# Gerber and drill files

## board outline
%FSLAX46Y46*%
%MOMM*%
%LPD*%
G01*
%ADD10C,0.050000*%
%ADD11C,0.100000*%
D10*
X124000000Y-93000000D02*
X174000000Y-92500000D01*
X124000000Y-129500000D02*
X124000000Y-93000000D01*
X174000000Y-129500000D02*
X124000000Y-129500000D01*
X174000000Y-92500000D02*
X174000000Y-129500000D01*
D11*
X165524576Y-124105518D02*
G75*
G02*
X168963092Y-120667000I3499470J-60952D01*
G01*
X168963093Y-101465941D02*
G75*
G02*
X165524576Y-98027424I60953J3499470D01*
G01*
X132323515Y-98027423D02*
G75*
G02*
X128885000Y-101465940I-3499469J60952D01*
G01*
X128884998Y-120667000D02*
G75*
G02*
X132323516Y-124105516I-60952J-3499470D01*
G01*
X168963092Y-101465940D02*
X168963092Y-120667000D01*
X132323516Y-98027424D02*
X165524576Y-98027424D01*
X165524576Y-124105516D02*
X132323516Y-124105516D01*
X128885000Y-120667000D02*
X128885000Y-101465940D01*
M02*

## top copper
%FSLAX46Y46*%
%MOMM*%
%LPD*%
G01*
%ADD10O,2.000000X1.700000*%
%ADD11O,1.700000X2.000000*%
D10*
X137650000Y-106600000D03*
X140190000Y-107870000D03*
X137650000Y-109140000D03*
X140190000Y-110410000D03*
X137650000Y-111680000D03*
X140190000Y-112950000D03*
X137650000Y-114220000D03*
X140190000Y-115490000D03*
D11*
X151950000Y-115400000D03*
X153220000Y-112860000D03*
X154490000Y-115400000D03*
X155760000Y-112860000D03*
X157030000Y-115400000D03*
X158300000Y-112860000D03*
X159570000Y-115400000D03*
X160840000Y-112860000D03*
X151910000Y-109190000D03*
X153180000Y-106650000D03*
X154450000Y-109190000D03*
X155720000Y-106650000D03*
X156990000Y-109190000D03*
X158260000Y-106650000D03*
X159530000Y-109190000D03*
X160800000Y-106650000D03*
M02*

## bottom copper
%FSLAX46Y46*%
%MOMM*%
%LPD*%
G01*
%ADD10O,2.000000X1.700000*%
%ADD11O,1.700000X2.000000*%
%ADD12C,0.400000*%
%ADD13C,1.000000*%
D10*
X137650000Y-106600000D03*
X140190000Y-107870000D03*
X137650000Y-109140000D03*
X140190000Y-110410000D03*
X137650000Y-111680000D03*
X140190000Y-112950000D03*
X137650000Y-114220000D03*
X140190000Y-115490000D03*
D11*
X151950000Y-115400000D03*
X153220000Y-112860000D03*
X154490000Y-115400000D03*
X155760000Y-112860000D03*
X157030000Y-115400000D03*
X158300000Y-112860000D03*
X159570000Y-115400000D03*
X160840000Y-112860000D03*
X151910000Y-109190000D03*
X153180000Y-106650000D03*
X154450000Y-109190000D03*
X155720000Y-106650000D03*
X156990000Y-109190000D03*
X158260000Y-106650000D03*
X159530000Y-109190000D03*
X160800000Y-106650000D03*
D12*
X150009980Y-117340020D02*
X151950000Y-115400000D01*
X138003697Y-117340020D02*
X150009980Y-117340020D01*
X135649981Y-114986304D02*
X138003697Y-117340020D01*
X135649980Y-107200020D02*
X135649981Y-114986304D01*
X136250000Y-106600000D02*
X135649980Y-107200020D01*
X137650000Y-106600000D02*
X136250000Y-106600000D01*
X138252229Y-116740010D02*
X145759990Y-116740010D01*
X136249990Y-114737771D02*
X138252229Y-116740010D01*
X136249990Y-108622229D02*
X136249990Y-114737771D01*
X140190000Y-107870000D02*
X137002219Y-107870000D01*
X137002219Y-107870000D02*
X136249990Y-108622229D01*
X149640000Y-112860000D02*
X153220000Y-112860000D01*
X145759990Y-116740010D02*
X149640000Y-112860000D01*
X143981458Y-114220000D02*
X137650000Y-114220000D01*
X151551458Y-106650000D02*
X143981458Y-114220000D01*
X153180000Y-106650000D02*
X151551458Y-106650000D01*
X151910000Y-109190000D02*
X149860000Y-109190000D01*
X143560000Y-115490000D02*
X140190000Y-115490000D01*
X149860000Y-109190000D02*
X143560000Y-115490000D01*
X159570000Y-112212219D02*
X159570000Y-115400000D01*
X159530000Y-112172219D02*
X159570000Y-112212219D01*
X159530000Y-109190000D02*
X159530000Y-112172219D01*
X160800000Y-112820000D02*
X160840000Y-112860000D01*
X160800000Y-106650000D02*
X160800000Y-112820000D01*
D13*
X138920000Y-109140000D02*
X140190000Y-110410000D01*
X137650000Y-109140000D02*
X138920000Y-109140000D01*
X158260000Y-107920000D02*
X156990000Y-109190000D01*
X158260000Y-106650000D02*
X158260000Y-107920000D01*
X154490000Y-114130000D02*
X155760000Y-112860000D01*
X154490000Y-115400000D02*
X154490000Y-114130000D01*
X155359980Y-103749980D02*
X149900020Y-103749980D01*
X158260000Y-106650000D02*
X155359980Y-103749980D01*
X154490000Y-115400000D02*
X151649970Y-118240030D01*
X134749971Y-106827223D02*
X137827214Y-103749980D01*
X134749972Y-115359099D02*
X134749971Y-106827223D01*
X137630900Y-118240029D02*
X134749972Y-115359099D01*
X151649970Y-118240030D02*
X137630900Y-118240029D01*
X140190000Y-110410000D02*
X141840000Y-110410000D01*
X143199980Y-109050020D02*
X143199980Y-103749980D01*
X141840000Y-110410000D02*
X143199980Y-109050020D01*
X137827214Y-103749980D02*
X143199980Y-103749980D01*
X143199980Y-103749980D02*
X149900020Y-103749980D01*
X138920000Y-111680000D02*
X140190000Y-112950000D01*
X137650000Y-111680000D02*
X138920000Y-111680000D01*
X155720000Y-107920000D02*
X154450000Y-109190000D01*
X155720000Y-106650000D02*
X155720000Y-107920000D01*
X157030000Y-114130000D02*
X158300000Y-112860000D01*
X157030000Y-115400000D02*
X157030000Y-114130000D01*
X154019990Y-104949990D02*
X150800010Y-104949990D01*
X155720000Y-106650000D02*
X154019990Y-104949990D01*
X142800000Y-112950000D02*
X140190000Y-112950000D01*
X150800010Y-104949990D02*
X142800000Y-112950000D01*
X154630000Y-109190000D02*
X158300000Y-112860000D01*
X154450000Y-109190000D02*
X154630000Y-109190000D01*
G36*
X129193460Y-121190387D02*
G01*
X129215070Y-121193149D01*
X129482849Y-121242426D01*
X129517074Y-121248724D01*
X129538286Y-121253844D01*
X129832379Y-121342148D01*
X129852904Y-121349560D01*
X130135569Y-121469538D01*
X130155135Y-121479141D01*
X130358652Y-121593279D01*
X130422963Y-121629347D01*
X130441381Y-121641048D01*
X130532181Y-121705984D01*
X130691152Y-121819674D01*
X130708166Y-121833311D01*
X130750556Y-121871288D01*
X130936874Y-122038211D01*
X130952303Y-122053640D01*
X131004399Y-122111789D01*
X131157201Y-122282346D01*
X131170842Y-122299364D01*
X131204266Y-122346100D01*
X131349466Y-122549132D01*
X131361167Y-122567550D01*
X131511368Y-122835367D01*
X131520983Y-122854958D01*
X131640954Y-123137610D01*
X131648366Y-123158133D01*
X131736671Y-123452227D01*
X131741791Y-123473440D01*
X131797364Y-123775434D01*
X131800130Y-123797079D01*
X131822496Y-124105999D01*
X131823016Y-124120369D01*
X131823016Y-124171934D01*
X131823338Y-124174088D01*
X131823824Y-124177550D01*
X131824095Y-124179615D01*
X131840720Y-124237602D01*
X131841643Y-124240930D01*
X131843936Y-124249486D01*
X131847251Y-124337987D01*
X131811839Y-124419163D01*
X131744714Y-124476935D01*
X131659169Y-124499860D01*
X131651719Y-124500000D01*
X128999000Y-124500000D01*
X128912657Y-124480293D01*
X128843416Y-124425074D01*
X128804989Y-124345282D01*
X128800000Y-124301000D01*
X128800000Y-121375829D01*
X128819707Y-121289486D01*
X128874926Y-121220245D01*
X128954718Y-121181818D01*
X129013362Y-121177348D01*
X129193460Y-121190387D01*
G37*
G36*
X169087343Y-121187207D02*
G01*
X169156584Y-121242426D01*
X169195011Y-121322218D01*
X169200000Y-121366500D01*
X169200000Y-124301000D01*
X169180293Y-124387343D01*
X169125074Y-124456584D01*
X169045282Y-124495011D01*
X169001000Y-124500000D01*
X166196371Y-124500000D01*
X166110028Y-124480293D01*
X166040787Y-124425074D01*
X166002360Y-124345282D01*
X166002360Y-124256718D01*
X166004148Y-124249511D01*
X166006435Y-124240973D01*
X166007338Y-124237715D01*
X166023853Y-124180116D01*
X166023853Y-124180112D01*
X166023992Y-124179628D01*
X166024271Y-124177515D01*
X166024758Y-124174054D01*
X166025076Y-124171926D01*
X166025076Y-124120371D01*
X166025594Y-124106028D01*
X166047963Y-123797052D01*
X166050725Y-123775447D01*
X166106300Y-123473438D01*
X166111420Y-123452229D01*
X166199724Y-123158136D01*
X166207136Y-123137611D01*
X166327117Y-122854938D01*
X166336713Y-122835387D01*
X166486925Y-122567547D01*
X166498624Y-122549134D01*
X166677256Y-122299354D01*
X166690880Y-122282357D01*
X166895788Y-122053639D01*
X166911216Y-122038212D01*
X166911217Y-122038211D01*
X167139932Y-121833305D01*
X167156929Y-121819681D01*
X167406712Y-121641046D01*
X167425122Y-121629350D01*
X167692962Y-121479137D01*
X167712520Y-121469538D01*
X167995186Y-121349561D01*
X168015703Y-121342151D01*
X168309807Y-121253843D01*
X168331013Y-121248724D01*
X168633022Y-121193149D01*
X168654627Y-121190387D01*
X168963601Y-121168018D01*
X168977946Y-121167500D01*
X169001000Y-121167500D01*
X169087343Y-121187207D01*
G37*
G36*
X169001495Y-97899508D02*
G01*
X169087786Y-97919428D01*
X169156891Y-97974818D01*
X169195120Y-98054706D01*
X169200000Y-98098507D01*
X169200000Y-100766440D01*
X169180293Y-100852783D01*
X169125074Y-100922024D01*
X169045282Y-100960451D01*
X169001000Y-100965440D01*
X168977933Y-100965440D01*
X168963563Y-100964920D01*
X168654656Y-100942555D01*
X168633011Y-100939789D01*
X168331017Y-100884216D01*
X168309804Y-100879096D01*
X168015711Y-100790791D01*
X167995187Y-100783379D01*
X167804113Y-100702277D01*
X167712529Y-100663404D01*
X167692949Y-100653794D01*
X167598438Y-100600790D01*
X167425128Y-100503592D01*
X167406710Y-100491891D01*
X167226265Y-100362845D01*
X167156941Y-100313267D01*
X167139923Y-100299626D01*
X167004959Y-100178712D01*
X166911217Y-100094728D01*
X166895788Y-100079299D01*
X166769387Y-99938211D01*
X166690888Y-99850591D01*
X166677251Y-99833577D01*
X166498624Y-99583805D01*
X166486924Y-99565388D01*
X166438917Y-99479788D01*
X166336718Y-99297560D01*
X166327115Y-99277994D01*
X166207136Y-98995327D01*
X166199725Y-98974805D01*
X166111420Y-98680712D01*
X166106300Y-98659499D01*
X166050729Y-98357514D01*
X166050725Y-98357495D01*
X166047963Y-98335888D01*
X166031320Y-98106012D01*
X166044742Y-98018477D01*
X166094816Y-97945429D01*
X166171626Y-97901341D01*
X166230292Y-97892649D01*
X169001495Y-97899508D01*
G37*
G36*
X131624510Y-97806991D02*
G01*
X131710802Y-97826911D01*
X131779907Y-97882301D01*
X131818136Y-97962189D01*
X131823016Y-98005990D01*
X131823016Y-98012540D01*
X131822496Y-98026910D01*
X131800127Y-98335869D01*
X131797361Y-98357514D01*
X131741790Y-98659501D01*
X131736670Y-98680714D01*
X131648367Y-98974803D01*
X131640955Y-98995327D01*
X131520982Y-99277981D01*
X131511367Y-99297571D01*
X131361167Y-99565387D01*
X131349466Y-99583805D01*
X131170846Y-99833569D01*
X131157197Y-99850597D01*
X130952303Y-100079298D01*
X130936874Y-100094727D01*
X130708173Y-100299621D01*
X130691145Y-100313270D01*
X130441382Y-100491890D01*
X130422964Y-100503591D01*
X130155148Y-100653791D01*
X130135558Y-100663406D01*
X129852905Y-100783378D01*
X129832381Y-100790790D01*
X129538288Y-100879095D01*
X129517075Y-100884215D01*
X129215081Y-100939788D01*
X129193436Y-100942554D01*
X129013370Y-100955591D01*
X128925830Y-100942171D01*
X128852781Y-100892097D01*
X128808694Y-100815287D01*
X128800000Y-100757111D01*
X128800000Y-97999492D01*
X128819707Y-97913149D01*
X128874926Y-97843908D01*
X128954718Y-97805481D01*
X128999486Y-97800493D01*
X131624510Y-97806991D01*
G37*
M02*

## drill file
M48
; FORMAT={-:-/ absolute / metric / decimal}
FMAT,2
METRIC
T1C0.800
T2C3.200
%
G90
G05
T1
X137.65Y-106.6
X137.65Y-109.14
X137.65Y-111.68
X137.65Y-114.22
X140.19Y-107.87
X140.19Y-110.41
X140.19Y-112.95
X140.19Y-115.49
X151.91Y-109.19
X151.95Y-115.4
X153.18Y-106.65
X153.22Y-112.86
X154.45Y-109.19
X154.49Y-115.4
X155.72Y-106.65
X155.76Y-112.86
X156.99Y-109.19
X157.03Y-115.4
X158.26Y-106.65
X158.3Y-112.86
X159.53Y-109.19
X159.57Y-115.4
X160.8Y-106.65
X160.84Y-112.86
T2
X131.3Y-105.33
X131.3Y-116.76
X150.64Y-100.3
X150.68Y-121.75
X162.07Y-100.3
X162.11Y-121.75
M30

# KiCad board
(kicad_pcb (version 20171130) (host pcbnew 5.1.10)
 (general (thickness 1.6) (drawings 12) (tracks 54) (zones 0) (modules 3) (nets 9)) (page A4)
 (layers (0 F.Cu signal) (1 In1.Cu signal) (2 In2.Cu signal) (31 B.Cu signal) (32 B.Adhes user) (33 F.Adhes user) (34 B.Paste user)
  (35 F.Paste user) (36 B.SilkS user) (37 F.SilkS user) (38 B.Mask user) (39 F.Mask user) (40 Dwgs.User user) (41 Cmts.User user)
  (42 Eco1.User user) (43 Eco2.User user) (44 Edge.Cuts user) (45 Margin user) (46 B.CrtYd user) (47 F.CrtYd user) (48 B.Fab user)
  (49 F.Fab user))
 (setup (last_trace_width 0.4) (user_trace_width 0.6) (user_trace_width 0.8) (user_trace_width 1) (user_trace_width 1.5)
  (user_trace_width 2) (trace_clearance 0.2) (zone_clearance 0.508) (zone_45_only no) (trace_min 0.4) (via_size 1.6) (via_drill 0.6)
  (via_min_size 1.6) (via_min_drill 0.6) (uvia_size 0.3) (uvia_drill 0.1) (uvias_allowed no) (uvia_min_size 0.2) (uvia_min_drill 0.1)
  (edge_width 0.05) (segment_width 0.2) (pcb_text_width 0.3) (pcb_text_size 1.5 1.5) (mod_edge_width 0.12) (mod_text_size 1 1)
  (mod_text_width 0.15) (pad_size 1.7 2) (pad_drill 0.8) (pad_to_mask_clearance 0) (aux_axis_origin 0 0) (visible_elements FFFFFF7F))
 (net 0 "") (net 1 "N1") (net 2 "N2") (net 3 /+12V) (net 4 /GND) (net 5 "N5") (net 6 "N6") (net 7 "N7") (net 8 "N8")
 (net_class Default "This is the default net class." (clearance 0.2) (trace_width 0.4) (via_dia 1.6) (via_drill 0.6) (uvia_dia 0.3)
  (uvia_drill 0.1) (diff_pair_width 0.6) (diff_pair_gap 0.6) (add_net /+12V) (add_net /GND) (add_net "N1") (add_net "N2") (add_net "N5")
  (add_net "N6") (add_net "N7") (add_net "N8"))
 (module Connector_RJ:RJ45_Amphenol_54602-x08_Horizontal (layer F.Cu) (at 137.65 106.6 270)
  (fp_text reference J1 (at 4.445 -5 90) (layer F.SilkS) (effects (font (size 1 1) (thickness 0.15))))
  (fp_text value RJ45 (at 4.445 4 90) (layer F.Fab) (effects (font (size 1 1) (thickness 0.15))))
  (pad "" np_thru_hole circle (at 10.16 6.35 270) (size 3.2 3.2) (drill 3.2) (layers *.Cu *.Mask))
  (pad "" np_thru_hole circle (at -1.27 6.35 270) (size 3.2 3.2) (drill 3.2) (layers *.Cu *.Mask))
  (pad 1 thru_hole oval (at 0 0 270) (size 1.7 2) (drill 0.8) (layers *.Cu *.Mask) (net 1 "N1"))
  (pad 2 thru_hole oval (at 1.27 -2.54 270) (size 1.7 2) (drill 0.8) (layers *.Cu *.Mask) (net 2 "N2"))
  (pad 3 thru_hole oval (at 2.54 0 270) (size 1.7 2) (drill 0.8) (layers *.Cu *.Mask) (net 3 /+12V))
  (pad 4 thru_hole oval (at 3.81 -2.54 270) (size 1.7 2) (drill 0.8) (layers *.Cu *.Mask) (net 3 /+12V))
  (pad 5 thru_hole oval (at 5.08 0 270) (size 1.7 2) (drill 0.8) (layers *.Cu *.Mask) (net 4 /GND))
  (pad 6 thru_hole oval (at 6.35 -2.54 270) (size 1.7 2) (drill 0.8) (layers *.Cu *.Mask) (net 4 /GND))
  (pad 7 thru_hole oval (at 7.62 0 270) (size 1.7 2) (drill 0.8) (layers *.Cu *.Mask) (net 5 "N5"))
  (pad 8 thru_hole oval (at 8.89 -2.54 270) (size 1.7 2) (drill 0.8) (layers *.Cu *.Mask) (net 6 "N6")))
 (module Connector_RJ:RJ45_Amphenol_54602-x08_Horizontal (layer F.Cu) (at 151.95 115.4)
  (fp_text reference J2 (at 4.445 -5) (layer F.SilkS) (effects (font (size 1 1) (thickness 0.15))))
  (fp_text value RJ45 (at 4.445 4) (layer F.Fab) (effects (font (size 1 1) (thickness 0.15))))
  (pad "" np_thru_hole circle (at 10.16 6.35) (size 3.2 3.2) (drill 3.2) (layers *.Cu *.Mask))
  (pad "" np_thru_hole circle (at -1.27 6.35) (size 3.2 3.2) (drill 3.2) (layers *.Cu *.Mask))
  (pad 1 thru_hole oval (at 0 0) (size 1.7 2) (drill 0.8) (layers *.Cu *.Mask) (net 1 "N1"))
  (pad 2 thru_hole oval (at 1.27 -2.54) (size 1.7 2) (drill 0.8) (layers *.Cu *.Mask) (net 2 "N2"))
  (pad 3 thru_hole oval (at 2.54 0) (size 1.7 2) (drill 0.8) (layers *.Cu *.Mask) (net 3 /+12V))
  (pad 4 thru_hole oval (at 3.81 -2.54) (size 1.7 2) (drill 0.8) (layers *.Cu *.Mask) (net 3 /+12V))
  (pad 5 thru_hole oval (at 5.08 0) (size 1.7 2) (drill 0.8) (layers *.Cu *.Mask) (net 4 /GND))
  (pad 6 thru_hole oval (at 6.35 -2.54) (size 1.7 2) (drill 0.8) (layers *.Cu *.Mask) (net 4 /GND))
  (pad 7 thru_hole oval (at 7.62 0) (size 1.7 2) (drill 0.8) (layers *.Cu *.Mask) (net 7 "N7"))
  (pad 8 thru_hole oval (at 8.89 -2.54) (size 1.7 2) (drill 0.8) (layers *.Cu *.Mask) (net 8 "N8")))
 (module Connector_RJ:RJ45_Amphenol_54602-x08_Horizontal (layer F.Cu) (at 160.8 106.65 180)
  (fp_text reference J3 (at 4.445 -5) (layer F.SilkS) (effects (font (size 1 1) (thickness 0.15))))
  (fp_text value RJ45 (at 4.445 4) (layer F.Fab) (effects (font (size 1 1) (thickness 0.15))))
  (pad 8 thru_hole oval (at 8.89 -2.54 180) (size 1.7 2) (drill 0.8) (layers *.Cu *.Mask) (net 6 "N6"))
  (pad 7 thru_hole oval (at 7.62 0 180) (size 1.7 2) (drill 0.8) (layers *.Cu *.Mask) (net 5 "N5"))
  (pad 6 thru_hole oval (at 6.35 -2.54 180) (size 1.7 2) (drill 0.8) (layers *.Cu *.Mask) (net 4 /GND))
  (pad 5 thru_hole oval (at 5.08 0 180) (size 1.7 2) (drill 0.8) (layers *.Cu *.Mask) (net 4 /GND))
  (pad 4 thru_hole oval (at 3.81 -2.54 180) (size 1.7 2) (drill 0.8) (layers *.Cu *.Mask) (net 3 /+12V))
  (pad 3 thru_hole oval (at 2.54 0 180) (size 1.7 2) (drill 0.8) (layers *.Cu *.Mask) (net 3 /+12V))
  (pad 2 thru_hole oval (at 1.27 -2.54 180) (size 1.7 2) (drill 0.8) (layers *.Cu *.Mask) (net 7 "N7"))
  (pad 1 thru_hole oval (at 0 0 180) (size 1.7 2) (drill 0.8) (layers *.Cu *.Mask) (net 8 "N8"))
  (pad "" np_thru_hole circle (at -1.27 6.35 180) (size 3.2 3.2) (drill 3.2) (layers *.Cu *.Mask))
  (pad "" np_thru_hole circle (at 10.16 6.35 180) (size 3.2 3.2) (drill 3.2) (layers *.Cu *.Mask)))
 (gr_line (start 124 93) (end 174 92.5) (layer Edge.Cuts) (width 0.05))
 (gr_line (start 124 129.5) (end 124 93) (layer Edge.Cuts) (width 0.05))
 (gr_line (start 174 129.5) (end 124 129.5) (layer Edge.Cuts) (width 0.05))
 (gr_line (start 174 92.5) (end 174 129.5) (layer Edge.Cuts) (width 0.05))
 (gr_arc (start 169.024046 124.16647) (end 168.963092 120.667) (angle -88.00426351) (layer Edge.Cuts) (width 0.1))
 (gr_arc (start 169.024046 97.966471) (end 165.524576 98.027424) (angle -88.00426351) (layer Edge.Cuts) (width 0.1))
 (gr_arc (start 128.824046 97.966471) (end 128.885 101.46594) (angle -88.00426351) (layer Edge.Cuts) (width 0.1))
 (gr_arc (start 128.824046 124.16647) (end 132.323516 124.105516) (angle -88.00426351) (layer Edge.Cuts) (width 0.1))
 (gr_line (start 168.963092 101.46594) (end 168.963092 120.667) (layer Edge.Cuts) (width 0.1))
 (gr_line (start 132.323516 98.027424) (end 165.524576 98.027424) (layer Edge.Cuts) (width 0.1))
 (gr_line (start 165.524576 124.105516) (end 132.323516 124.105516) (layer Edge.Cuts) (width 0.1))
 (gr_line (start 128.885 120.667) (end 128.885 101.46594) (layer Edge.Cuts) (width 0.1))
 (segment (start 150.00998 117.34002) (end 151.95 115.4) (width 0.4) (layer B.Cu) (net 1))
 (segment (start 138.003697 117.34002) (end 150.00998 117.34002) (width 0.4) (layer B.Cu) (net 1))
 (segment (start 135.649981 114.986304) (end 138.003697 117.34002) (width 0.4) (layer B.Cu) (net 1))
 (segment (start 135.64998 107.20002) (end 135.649981 114.986304) (width 0.4) (layer B.Cu) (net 1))
 (segment (start 136.25 106.6) (end 135.64998 107.20002) (width 0.4) (layer B.Cu) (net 1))
 (segment (start 137.65 106.6) (end 136.25 106.6) (width 0.4) (layer B.Cu) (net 1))
 (segment (start 138.252229 116.74001) (end 145.75999 116.74001) (width 0.4) (layer B.Cu) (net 2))
 (segment (start 136.24999 114.737771) (end 138.252229 116.74001) (width 0.4) (layer B.Cu) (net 2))
 (segment (start 136.24999 108.622229) (end 136.24999 114.737771) (width 0.4) (layer B.Cu) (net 2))
 (segment (start 140.19 107.87) (end 137.002219 107.87) (width 0.4) (layer B.Cu) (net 2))
 (segment (start 137.002219 107.87) (end 136.24999 108.622229) (width 0.4) (layer B.Cu) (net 2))
 (segment (start 149.64 112.86) (end 153.22 112.86) (width 0.4) (layer B.Cu) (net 2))
 (segment (start 145.75999 116.74001) (end 149.64 112.86) (width 0.4) (layer B.Cu) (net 2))
 (segment (start 143.981458 114.22) (end 137.65 114.22) (width 0.4) (layer B.Cu) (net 5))
 (segment (start 151.551458 106.65) (end 143.981458 114.22) (width 0.4) (layer B.Cu) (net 5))
 (segment (start 153.18 106.65) (end 151.551458 106.65) (width 0.4) (layer B.Cu) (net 5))
 (segment (start 151.91 109.19) (end 149.86 109.19) (width 0.4) (layer B.Cu) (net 6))
 (segment (start 143.56 115.49) (end 140.19 115.49) (width 0.4) (layer B.Cu) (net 6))
 (segment (start 149.86 109.19) (end 143.56 115.49) (width 0.4) (layer B.Cu) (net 6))
 (segment (start 159.57 112.212219) (end 159.57 115.4) (width 0.4) (layer B.Cu) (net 7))
 (segment (start 159.53 112.172219) (end 159.57 112.212219) (width 0.4) (layer B.Cu) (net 7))
 (segment (start 159.53 109.19) (end 159.53 112.172219) (width 0.4) (layer B.Cu) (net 7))
 (segment (start 160.8 112.82) (end 160.84 112.86) (width 0.4) (layer B.Cu) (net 8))
 (segment (start 160.8 106.65) (end 160.8 112.82) (width 0.4) (layer B.Cu) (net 8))
 (segment (start 138.92 109.14) (end 140.19 110.41) (width 1) (layer B.Cu) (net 3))
 (segment (start 137.65 109.14) (end 138.92 109.14) (width 1) (layer B.Cu) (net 3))
 (segment (start 158.26 107.92) (end 156.99 109.19) (width 1) (layer B.Cu) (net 3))
 (segment (start 158.26 106.65) (end 158.26 107.92) (width 1) (layer B.Cu) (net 3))
 (segment (start 154.49 114.13) (end 155.76 112.86) (width 1) (layer B.Cu) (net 3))
 (segment (start 154.49 115.4) (end 154.49 114.13) (width 1) (layer B.Cu) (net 3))
 (segment (start 155.35998 103.74998) (end 149.90002 103.74998) (width 1) (layer B.Cu) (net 3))
 (segment (start 158.26 106.65) (end 155.35998 103.74998) (width 1) (layer B.Cu) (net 3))
 (segment (start 154.49 115.4) (end 151.64997 118.24003) (width 1) (layer B.Cu) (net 3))
 (segment (start 134.749971 106.827223) (end 137.827214 103.74998) (width 1) (layer B.Cu) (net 3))
 (segment (start 134.749972 115.359099) (end 134.749971 106.827223) (width 1) (layer B.Cu) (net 3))
 (segment (start 137.6309 118.240029) (end 134.749972 115.359099) (width 1) (layer B.Cu) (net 3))
 (segment (start 151.64997 118.24003) (end 137.6309 118.240029) (width 1) (layer B.Cu) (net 3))
 (segment (start 140.19 110.41) (end 141.84 110.41) (width 1) (layer B.Cu) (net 3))
 (segment (start 143.19998 109.05002) (end 143.19998 103.74998) (width 1) (layer B.Cu) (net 3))
 (segment (start 141.84 110.41) (end 143.19998 109.05002) (width 1) (layer B.Cu) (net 3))
 (segment (start 137.827214 103.74998) (end 143.19998 103.74998) (width 1) (layer B.Cu) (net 3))
 (segment (start 143.19998 103.74998) (end 149.90002 103.74998) (width 1) (layer B.Cu) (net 3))
 (segment (start 138.92 111.68) (end 140.19 112.95) (width 1) (layer B.Cu) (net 4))
 (segment (start 137.65 111.68) (end 138.92 111.68) (width 1) (layer B.Cu) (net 4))
 (segment (start 155.72 107.92) (end 154.45 109.19) (width 1) (layer B.Cu) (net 4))
 (segment (start 155.72 106.65) (end 155.72 107.92) (width 1) (layer B.Cu) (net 4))
 (segment (start 157.03 114.13) (end 158.3 112.86) (width 1) (layer B.Cu) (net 4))
 (segment (start 157.03 115.4) (end 157.03 114.13) (width 1) (layer B.Cu) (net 4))
 (segment (start 154.01999 104.94999) (end 150.80001 104.94999) (width 1) (layer B.Cu) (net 4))
 (segment (start 155.72 106.65) (end 154.01999 104.94999) (width 1) (layer B.Cu) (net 4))
 (segment (start 142.8 112.95) (end 140.19 112.95) (width 1) (layer B.Cu) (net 4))
 (segment (start 150.80001 104.94999) (end 142.8 112.95) (width 1) (layer B.Cu) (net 4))
 (segment (start 154.63 109.19) (end 158.3 112.86) (width 1) (layer B.Cu) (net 4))
 (segment (start 154.45 109.19) (end 154.63 109.19) (width 1) (layer B.Cu) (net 4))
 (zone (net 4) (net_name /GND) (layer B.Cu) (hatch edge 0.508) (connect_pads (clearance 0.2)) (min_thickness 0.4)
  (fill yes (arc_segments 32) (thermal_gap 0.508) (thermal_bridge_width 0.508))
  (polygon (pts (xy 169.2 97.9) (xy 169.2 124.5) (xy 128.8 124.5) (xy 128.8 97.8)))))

